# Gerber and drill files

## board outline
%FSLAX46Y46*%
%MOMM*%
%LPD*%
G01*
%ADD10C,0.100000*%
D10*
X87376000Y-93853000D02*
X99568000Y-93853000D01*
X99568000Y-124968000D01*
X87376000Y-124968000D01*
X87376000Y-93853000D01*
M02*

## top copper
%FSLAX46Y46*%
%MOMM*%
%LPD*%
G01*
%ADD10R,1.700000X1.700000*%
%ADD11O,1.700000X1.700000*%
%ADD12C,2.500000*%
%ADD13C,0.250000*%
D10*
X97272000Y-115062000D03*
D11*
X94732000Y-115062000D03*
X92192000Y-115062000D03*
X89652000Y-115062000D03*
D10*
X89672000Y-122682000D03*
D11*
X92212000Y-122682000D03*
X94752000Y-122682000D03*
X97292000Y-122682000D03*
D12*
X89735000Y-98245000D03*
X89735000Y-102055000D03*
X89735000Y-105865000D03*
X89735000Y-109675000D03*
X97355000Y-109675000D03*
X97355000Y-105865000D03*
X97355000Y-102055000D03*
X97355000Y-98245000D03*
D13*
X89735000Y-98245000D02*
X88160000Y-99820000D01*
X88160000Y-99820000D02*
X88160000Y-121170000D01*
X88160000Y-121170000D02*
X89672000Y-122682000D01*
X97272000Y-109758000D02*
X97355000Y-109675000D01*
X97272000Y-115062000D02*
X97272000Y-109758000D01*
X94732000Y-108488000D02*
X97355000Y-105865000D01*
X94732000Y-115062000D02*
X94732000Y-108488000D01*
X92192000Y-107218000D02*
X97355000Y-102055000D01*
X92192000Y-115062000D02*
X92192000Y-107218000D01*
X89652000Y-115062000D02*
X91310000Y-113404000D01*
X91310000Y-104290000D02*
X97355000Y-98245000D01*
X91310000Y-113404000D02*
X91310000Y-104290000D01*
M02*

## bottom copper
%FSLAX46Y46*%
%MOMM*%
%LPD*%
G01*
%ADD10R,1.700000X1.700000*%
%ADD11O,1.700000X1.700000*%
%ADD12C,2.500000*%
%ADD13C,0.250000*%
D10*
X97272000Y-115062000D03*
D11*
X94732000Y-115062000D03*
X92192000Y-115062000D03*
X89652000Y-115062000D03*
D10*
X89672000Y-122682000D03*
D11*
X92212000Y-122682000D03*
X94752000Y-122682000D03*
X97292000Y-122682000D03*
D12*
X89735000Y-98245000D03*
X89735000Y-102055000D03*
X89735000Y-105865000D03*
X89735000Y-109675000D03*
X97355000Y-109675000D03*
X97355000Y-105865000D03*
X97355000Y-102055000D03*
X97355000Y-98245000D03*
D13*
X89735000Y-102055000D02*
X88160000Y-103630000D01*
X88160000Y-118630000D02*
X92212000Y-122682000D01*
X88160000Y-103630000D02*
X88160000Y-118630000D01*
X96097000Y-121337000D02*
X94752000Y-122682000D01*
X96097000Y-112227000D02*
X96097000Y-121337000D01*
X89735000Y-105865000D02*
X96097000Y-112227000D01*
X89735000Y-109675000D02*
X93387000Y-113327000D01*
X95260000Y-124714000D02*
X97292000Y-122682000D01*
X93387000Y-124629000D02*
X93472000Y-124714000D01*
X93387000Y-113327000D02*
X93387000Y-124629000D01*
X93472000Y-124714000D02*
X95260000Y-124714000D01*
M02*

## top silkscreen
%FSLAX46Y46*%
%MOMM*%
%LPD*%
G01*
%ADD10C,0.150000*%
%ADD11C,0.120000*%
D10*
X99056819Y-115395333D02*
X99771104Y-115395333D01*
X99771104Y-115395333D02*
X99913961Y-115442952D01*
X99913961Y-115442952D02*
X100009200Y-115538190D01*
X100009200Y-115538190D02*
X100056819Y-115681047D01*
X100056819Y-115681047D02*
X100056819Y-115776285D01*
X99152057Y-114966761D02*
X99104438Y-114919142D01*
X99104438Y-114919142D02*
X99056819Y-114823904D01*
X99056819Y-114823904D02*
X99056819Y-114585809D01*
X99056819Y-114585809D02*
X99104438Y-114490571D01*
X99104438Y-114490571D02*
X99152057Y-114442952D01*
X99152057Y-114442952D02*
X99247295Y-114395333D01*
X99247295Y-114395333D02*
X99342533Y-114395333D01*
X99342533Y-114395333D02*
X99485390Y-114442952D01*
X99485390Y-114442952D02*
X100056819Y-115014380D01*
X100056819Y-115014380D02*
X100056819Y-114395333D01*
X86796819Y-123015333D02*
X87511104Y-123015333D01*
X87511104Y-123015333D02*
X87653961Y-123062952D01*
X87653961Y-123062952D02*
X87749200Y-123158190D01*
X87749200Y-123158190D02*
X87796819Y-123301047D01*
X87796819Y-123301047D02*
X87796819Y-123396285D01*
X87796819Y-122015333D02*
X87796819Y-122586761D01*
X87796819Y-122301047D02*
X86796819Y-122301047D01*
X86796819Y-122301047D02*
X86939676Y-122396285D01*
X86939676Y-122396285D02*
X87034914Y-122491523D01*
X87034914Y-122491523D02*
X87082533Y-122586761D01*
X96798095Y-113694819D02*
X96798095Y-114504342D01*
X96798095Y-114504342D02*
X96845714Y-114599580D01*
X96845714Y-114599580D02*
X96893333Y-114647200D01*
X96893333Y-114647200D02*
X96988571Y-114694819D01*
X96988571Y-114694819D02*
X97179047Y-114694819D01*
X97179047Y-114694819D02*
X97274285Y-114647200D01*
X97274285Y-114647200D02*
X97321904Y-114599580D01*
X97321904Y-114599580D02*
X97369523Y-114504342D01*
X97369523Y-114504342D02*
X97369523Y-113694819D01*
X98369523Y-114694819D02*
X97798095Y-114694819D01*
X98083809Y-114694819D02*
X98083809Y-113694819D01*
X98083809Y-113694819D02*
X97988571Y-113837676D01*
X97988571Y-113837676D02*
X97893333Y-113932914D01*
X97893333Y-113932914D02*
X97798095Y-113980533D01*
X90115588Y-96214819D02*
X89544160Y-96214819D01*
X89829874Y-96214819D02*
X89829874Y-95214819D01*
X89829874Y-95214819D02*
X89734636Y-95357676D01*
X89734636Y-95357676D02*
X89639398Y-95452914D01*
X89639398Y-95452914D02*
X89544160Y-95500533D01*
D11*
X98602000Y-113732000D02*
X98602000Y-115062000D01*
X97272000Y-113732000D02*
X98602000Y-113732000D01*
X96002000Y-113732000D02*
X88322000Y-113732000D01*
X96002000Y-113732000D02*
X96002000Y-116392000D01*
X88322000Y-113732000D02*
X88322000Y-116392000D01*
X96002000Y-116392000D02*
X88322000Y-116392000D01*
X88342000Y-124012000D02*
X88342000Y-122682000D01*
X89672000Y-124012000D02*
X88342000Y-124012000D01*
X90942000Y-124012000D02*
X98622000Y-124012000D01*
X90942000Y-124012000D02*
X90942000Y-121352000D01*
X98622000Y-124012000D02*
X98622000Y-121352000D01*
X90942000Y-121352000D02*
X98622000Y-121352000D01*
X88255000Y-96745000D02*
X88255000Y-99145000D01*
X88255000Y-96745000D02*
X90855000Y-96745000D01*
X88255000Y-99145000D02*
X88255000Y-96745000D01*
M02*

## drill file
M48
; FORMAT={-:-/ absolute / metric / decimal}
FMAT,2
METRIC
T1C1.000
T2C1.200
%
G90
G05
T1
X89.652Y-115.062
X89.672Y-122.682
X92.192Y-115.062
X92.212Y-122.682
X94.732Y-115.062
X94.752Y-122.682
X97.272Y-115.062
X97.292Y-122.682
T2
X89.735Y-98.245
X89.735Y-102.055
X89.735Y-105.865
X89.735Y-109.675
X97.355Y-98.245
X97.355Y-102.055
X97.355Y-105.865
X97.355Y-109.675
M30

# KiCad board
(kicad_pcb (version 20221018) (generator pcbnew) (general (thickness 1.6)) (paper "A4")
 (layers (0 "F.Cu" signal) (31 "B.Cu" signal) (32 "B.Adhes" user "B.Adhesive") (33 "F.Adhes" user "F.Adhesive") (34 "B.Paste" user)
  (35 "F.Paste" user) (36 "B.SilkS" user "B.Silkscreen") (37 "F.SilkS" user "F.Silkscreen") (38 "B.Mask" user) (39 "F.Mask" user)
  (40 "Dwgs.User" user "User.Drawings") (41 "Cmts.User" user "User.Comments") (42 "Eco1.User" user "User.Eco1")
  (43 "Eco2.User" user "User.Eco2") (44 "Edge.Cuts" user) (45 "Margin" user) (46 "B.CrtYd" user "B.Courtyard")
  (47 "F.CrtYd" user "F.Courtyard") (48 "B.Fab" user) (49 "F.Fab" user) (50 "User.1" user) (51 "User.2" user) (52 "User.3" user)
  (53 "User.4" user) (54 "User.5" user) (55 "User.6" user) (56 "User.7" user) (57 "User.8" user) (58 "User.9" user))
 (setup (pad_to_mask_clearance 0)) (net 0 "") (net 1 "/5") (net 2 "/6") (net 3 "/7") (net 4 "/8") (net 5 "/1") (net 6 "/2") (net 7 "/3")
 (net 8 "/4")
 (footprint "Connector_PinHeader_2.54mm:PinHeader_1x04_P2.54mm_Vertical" (layer "F.Cu") (at 97.272 115.062 -90)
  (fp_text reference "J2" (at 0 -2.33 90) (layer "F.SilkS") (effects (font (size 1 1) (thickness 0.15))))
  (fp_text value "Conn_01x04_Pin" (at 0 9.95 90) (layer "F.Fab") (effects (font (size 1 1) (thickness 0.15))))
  (fp_line (start -1.33 -1.33) (end 0 -1.33) (stroke (width 0.12) (type solid)) (layer "F.SilkS"))
  (fp_line (start -1.33 0) (end -1.33 -1.33) (stroke (width 0.12) (type solid)) (layer "F.SilkS"))
  (fp_line (start -1.33 1.27) (end -1.33 8.95) (stroke (width 0.12) (type solid)) (layer "F.SilkS"))
  (fp_line (start -1.33 1.27) (end 1.33 1.27) (stroke (width 0.12) (type solid)) (layer "F.SilkS"))
  (fp_line (start -1.33 8.95) (end 1.33 8.95) (stroke (width 0.12) (type solid)) (layer "F.SilkS"))
  (fp_line (start 1.33 1.27) (end 1.33 8.95) (stroke (width 0.12) (type solid)) (layer "F.SilkS"))
  (pad "1" thru_hole rect (at 0 0 270) (size 1.7 1.7) (drill 1) (layers "*.Cu" "*.Mask") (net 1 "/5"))
  (pad "2" thru_hole oval (at 0 2.54 270) (size 1.7 1.7) (drill 1) (layers "*.Cu" "*.Mask") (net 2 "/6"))
  (pad "3" thru_hole oval (at 0 5.08 270) (size 1.7 1.7) (drill 1) (layers "*.Cu" "*.Mask") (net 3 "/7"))
  (pad "4" thru_hole oval (at 0 7.62 270) (size 1.7 1.7) (drill 1) (layers "*.Cu" "*.Mask") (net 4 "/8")))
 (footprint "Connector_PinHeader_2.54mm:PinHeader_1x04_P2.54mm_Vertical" (layer "F.Cu") (at 89.672 122.682 90)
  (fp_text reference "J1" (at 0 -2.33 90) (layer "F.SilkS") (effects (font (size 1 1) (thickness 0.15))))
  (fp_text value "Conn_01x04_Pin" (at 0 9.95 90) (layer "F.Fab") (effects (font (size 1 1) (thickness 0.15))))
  (fp_line (start -1.33 -1.33) (end 0 -1.33) (stroke (width 0.12) (type solid)) (layer "F.SilkS"))
  (fp_line (start -1.33 0) (end -1.33 -1.33) (stroke (width 0.12) (type solid)) (layer "F.SilkS"))
  (fp_line (start -1.33 1.27) (end -1.33 8.95) (stroke (width 0.12) (type solid)) (layer "F.SilkS"))
  (fp_line (start -1.33 1.27) (end 1.33 1.27) (stroke (width 0.12) (type solid)) (layer "F.SilkS"))
  (fp_line (start -1.33 8.95) (end 1.33 8.95) (stroke (width 0.12) (type solid)) (layer "F.SilkS"))
  (fp_line (start 1.33 1.27) (end 1.33 8.95) (stroke (width 0.12) (type solid)) (layer "F.SilkS"))
  (pad "1" thru_hole rect (at 0 0 90) (size 1.7 1.7) (drill 1) (layers "*.Cu" "*.Mask") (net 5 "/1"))
  (pad "2" thru_hole oval (at 0 2.54 90) (size 1.7 1.7) (drill 1) (layers "*.Cu" "*.Mask") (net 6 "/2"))
  (pad "3" thru_hole oval (at 0 5.08 90) (size 1.7 1.7) (drill 1) (layers "*.Cu" "*.Mask") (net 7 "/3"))
  (pad "4" thru_hole oval (at 0 7.62 90) (size 1.7 1.7) (drill 1) (layers "*.Cu" "*.Mask") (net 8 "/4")))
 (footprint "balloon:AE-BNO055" (layer "F.Cu") (at 93.455 103.145)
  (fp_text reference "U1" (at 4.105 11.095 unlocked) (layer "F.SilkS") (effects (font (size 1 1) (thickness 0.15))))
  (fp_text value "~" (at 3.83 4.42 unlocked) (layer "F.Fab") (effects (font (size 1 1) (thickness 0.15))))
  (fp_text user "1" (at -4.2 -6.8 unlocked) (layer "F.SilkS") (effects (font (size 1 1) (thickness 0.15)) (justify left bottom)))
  (fp_line (start -5.2 -6.4) (end -5.2 -4) (stroke (width 0.12) (type default)) (layer "F.SilkS"))
  (fp_line (start -5.2 -6.4) (end -2.6 -6.4) (stroke (width 0.12) (type default)) (layer "F.SilkS"))
  (fp_line (start -5.2 -4) (end -5.2 -6.4) (stroke (width 0.12) (type default)) (layer "F.SilkS"))
  (pad "1" thru_hole circle (at -3.72 -4.9) (size 2.5 2.5) (drill 1.2) (layers "*.Cu" "*.Mask") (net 5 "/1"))
  (pad "2" thru_hole circle (at -3.72 -1.09) (size 2.5 2.5) (drill 1.2) (layers "*.Cu" "*.Mask") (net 6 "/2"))
  (pad "3" thru_hole circle (at -3.72 2.72) (size 2.5 2.5) (drill 1.2) (layers "*.Cu" "*.Mask") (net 7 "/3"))
  (pad "4" thru_hole circle (at -3.72 6.53) (size 2.5 2.5) (drill 1.2) (layers "*.Cu" "*.Mask") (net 8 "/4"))
  (pad "5" thru_hole circle (at 3.9 6.53) (size 2.5 2.5) (drill 1.2) (layers "*.Cu" "*.Mask") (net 1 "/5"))
  (pad "6" thru_hole circle (at 3.9 2.72) (size 2.5 2.5) (drill 1.2) (layers "*.Cu" "*.Mask") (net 2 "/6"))
  (pad "7" thru_hole circle (at 3.9 -1.09) (size 2.5 2.5) (drill 1.2) (layers "*.Cu" "*.Mask") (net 3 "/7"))
  (pad "8" thru_hole circle (at 3.9 -4.9) (size 2.5 2.5) (drill 1.2) (layers "*.Cu" "*.Mask") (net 4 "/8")))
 (gr_rect (start 87.376 93.853) (end 99.568 124.968) (stroke (width 0.1) (type default)) (fill none) (layer "Edge.Cuts"))
 (segment (start 89.735 98.245) (end 88.16 99.82) (width 0.25) (layer "F.Cu") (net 5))
 (segment (start 88.16 99.82) (end 88.16 121.17) (width 0.25) (layer "F.Cu") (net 5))
 (segment (start 88.16 121.17) (end 89.672 122.682) (width 0.25) (layer "F.Cu") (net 5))
 (segment (start 89.735 102.055) (end 88.16 103.63) (width 0.25) (layer "B.Cu") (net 6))
 (segment (start 88.16 118.63) (end 92.212 122.682) (width 0.25) (layer "B.Cu") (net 6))
 (segment (start 88.16 103.63) (end 88.16 118.63) (width 0.25) (layer "B.Cu") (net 6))
 (segment (start 96.097 121.337) (end 94.752 122.682) (width 0.25) (layer "B.Cu") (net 7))
 (segment (start 96.097 112.227) (end 96.097 121.337) (width 0.25) (layer "B.Cu") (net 7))
 (segment (start 89.735 105.865) (end 96.097 112.227) (width 0.25) (layer "B.Cu") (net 7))
 (segment (start 89.735 109.675) (end 93.387 113.327) (width 0.25) (layer "B.Cu") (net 8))
 (segment (start 95.26 124.714) (end 97.292 122.682) (width 0.25) (layer "B.Cu") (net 8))
 (segment (start 93.387 124.629) (end 93.472 124.714) (width 0.25) (layer "B.Cu") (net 8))
 (segment (start 93.387 113.327) (end 93.387 124.629) (width 0.25) (layer "B.Cu") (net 8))
 (segment (start 93.472 124.714) (end 95.26 124.714) (width 0.25) (layer "B.Cu") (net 8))
 (segment (start 97.272 109.758) (end 97.355 109.675) (width 0.25) (layer "F.Cu") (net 1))
 (segment (start 97.272 115.062) (end 97.272 109.758) (width 0.25) (layer "F.Cu") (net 1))
 (segment (start 94.732 108.488) (end 97.355 105.865) (width 0.25) (layer "F.Cu") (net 2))
 (segment (start 94.732 115.062) (end 94.732 108.488) (width 0.25) (layer "F.Cu") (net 2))
 (segment (start 92.192 107.218) (end 97.355 102.055) (width 0.25) (layer "F.Cu") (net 3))
 (segment (start 92.192 115.062) (end 92.192 107.218) (width 0.25) (layer "F.Cu") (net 3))
 (segment (start 89.652 115.062) (end 91.31 113.404) (width 0.25) (layer "F.Cu") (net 4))
 (segment (start 91.31 104.29) (end 97.355 98.245) (width 0.25) (layer "F.Cu") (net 4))
 (segment (start 91.31 113.404) (end 91.31 104.29) (width 0.25) (layer "F.Cu") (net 4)))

